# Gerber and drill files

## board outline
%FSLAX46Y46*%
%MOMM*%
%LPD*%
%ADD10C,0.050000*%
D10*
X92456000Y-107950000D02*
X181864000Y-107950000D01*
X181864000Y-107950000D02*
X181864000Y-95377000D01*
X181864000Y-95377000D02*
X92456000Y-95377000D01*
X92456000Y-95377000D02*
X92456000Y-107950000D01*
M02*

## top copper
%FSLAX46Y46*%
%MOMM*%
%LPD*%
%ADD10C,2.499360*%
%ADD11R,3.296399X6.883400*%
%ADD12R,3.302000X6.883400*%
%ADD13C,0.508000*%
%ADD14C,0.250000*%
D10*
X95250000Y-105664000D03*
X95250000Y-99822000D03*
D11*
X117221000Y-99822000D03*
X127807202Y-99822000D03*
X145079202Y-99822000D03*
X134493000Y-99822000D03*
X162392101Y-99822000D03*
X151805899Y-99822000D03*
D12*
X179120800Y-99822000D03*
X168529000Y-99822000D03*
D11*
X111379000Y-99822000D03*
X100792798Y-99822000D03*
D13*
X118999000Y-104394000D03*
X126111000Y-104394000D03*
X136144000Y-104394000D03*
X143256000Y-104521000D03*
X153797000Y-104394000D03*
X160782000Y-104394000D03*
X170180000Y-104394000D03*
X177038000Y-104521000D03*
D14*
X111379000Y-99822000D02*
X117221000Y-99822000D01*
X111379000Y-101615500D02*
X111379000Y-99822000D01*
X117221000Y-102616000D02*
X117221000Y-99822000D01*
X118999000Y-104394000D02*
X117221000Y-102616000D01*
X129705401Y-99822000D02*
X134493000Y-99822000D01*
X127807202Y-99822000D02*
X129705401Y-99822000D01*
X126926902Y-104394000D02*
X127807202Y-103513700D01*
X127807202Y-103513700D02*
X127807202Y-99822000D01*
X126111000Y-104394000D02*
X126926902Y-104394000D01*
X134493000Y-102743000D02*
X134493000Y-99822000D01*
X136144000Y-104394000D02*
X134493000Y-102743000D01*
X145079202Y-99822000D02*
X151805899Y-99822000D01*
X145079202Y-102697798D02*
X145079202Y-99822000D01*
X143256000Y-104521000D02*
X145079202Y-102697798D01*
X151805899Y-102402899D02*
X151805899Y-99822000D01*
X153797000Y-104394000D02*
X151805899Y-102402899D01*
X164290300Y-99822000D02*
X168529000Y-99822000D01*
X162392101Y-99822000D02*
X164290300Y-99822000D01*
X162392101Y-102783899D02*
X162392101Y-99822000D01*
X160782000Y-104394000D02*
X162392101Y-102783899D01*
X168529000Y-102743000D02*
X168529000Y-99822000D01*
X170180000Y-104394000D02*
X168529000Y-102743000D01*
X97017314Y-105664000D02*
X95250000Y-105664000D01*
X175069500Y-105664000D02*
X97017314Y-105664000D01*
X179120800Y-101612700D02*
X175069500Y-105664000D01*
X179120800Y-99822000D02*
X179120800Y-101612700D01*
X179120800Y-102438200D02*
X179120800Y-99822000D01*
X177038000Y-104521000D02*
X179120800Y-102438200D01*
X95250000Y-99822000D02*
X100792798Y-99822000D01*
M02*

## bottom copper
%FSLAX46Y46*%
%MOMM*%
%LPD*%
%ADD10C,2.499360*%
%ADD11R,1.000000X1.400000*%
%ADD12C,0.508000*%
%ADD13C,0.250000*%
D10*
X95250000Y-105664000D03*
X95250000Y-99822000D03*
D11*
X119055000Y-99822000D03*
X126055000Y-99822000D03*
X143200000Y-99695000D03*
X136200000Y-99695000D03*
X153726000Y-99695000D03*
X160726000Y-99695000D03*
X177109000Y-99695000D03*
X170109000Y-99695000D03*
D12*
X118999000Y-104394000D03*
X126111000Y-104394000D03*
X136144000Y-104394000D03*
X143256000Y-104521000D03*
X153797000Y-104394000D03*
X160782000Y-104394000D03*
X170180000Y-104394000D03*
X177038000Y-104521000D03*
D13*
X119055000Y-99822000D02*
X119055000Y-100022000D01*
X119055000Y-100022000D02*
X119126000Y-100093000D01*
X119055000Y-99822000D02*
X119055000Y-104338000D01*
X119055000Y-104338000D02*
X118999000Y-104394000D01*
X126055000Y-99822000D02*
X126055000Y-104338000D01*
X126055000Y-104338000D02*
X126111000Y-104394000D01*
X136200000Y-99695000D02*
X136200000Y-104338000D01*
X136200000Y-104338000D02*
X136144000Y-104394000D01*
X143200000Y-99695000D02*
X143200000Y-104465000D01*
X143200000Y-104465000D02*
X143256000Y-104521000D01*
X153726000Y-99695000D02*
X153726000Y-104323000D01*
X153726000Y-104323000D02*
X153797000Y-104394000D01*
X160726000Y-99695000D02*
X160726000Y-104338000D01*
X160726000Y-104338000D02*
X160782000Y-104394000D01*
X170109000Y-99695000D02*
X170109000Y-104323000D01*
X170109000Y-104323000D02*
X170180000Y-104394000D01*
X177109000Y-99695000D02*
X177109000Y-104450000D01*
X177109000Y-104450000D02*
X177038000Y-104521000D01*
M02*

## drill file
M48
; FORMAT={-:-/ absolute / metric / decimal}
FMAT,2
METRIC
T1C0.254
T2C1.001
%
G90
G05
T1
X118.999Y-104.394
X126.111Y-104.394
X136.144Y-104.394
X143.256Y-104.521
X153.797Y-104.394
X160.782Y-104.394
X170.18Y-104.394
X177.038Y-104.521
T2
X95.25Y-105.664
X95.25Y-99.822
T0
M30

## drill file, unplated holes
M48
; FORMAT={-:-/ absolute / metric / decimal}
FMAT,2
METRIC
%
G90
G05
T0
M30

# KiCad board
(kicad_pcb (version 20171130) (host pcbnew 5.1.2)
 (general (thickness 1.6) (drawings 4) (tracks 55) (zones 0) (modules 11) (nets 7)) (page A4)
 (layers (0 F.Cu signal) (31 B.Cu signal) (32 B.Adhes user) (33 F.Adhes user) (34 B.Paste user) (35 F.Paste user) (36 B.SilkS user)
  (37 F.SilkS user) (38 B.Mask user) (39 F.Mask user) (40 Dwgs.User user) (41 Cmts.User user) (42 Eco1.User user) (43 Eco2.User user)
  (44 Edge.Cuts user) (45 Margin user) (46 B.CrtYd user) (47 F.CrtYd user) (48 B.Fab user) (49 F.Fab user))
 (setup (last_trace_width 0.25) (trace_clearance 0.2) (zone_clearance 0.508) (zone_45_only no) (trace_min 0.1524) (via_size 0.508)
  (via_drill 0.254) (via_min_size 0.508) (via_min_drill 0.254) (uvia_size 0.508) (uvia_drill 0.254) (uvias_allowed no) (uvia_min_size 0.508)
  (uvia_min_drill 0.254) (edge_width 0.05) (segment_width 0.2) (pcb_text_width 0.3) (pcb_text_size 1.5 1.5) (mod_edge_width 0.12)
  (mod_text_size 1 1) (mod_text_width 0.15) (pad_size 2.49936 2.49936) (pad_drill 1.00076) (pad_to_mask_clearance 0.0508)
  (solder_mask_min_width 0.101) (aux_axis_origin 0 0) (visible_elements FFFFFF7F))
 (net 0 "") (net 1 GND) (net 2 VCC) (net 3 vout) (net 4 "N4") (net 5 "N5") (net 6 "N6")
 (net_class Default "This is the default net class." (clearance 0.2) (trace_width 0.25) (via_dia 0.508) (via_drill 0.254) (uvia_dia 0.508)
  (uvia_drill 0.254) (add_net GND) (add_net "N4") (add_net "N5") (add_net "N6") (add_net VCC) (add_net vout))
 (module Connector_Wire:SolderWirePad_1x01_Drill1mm (layer F.Cu) (at 95.25 105.664)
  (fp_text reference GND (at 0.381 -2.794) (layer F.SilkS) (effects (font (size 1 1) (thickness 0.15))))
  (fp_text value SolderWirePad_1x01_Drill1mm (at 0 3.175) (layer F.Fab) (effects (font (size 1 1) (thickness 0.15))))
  (pad 1 thru_hole circle (at 0 0) (size 2.49936 2.49936) (drill 1.00076) (layers *.Cu *.Mask) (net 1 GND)))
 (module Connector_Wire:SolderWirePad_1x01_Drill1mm (layer F.Cu) (at 95.25 99.822)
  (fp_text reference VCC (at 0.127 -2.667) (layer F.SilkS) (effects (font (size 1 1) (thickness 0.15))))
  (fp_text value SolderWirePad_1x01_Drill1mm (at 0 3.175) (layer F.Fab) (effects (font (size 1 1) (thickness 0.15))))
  (pad 1 thru_hole circle (at 0 0) (size 2.49936 2.49936) (drill 1.00076) (layers *.Cu *.Mask) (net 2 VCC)))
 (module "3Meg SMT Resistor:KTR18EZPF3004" (layer F.Cu) (at 122.514101 99.822 180)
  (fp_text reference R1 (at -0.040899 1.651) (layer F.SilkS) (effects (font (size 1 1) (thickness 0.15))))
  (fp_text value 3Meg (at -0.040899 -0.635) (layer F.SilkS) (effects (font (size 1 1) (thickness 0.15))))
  (pad 2 smd rect (at 5.293101 0 180) (size 3.296399 6.8834) (layers F.Cu F.Paste F.Mask) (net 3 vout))
  (pad 1 smd rect (at -5.293101 0 180) (size 3.296399 6.8834) (layers F.Cu F.Paste F.Mask) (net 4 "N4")))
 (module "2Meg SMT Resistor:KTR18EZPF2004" (layer F.Cu) (at 139.786101 99.822 180)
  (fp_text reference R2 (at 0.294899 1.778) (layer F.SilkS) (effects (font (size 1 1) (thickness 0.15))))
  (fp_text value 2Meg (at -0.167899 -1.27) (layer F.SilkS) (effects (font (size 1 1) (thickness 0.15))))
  (pad 1 smd rect (at -5.293101 0 180) (size 3.296399 6.8834) (layers F.Cu F.Paste F.Mask) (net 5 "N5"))
  (pad 2 smd rect (at 5.293101 0 180) (size 3.296399 6.8834) (layers F.Cu F.Paste F.Mask) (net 4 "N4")))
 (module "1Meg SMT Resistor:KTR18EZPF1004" (layer F.Cu) (at 157.099 99.822 180)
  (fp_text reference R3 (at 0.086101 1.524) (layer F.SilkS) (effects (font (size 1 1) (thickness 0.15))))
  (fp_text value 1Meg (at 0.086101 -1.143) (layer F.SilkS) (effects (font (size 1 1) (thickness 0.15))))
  (pad 1 smd rect (at -5.293101 0 180) (size 3.296399 6.8834) (layers F.Cu F.Paste F.Mask) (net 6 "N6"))
  (pad 2 smd rect (at 5.293101 0 180) (size 3.296399 6.8834) (layers F.Cu F.Paste F.Mask) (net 5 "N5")))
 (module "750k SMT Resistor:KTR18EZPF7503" (layer F.Cu) (at 173.8249 99.822 180)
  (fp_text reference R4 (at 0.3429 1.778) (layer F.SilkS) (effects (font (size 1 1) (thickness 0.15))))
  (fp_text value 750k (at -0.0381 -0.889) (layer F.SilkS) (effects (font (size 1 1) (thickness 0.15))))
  (pad 1 smd rect (at -5.2959 0 180) (size 3.302 6.8834) (layers F.Cu F.Paste F.Mask) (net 1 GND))
  (pad 2 smd rect (at 5.2959 0 180) (size 3.302 6.8834) (layers F.Cu F.Paste F.Mask) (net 6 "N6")))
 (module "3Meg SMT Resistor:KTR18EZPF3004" (layer F.Cu) (at 106.085899 99.822 180)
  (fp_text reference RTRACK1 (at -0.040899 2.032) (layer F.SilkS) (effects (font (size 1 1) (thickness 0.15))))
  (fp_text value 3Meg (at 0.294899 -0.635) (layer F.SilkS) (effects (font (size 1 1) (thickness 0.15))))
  (pad 1 smd rect (at -5.293101 0 180) (size 3.296399 6.8834) (layers F.Cu F.Paste F.Mask) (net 3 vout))
  (pad 2 smd rect (at 5.293101 0 180) (size 3.296399 6.8834) (layers F.Cu F.Paste F.Mask) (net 2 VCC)))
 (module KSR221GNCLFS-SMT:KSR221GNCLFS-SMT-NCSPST (layer B.Cu) (at 122.555 99.822)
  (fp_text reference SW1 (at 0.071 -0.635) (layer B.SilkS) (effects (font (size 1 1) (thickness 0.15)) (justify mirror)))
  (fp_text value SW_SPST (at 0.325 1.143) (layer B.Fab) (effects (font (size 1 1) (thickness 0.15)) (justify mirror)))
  (pad 1 smd rect (at -3.5 0) (size 1 1.4) (layers B.Cu B.Paste B.Mask) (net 3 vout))
  (pad 2 smd rect (at 3.5 0) (size 1 1.4) (layers B.Cu B.Paste B.Mask) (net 4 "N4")))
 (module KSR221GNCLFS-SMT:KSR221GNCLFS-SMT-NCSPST (layer B.Cu) (at 139.7 99.695)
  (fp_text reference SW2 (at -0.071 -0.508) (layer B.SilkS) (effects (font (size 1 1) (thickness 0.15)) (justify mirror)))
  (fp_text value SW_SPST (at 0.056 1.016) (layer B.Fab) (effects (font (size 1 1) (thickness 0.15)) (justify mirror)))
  (pad 2 smd rect (at 3.5 0) (size 1 1.4) (layers B.Cu B.Paste B.Mask) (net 5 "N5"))
  (pad 1 smd rect (at -3.5 0) (size 1 1.4) (layers B.Cu B.Paste B.Mask) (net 4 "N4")))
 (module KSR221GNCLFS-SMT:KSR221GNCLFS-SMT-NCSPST (layer B.Cu) (at 157.226 99.695)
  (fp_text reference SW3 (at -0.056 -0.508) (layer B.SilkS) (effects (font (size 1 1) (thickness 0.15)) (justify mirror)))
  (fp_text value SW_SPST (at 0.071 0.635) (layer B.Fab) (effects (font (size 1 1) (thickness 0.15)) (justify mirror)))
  (pad 1 smd rect (at -3.5 0) (size 1 1.4) (layers B.Cu B.Paste B.Mask) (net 5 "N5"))
  (pad 2 smd rect (at 3.5 0) (size 1 1.4) (layers B.Cu B.Paste B.Mask) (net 6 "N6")))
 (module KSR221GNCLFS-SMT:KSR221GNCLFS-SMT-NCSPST (layer B.Cu) (at 173.609 99.695)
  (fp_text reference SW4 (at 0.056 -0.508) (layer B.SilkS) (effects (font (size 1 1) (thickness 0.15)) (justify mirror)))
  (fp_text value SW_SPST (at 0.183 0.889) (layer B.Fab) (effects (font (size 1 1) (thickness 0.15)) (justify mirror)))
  (pad 2 smd rect (at 3.5 0) (size 1 1.4) (layers B.Cu B.Paste B.Mask) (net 1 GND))
  (pad 1 smd rect (at -3.5 0) (size 1 1.4) (layers B.Cu B.Paste B.Mask) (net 6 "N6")))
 (gr_line (start 92.456 107.95) (end 181.864 107.95) (layer Edge.Cuts) (width 0.05))
 (gr_line (start 181.864 107.95) (end 181.864 95.377) (layer Edge.Cuts) (width 0.05))
 (gr_line (start 181.864 95.377) (end 92.456 95.377) (layer Edge.Cuts) (width 0.05))
 (gr_line (start 92.456 95.377) (end 92.456 107.95) (layer Edge.Cuts) (width 0.05))
 (segment (start 111.379 99.822) (end 117.221 99.822) (width 0.25) (layer F.Cu) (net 3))
 (segment (start 119.055 99.822) (end 119.055 100.022) (width 0.25) (layer B.Cu) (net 3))
 (segment (start 119.055 100.022) (end 119.126 100.093) (width 0.25) (layer B.Cu) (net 3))
 (segment (start 111.379 101.6155) (end 111.379 99.822) (width 0.25) (layer F.Cu) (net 3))
 (via (at 118.999 104.394) (size 0.508) (drill 0.254) (layers F.Cu B.Cu) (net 3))
 (segment (start 119.055 99.822) (end 119.055 104.338) (width 0.25) (layer B.Cu) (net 3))
 (segment (start 119.055 104.338) (end 118.999 104.394) (width 0.25) (layer B.Cu) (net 3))
 (segment (start 117.221 102.616) (end 117.221 99.822) (width 0.25) (layer F.Cu) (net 3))
 (segment (start 118.999 104.394) (end 117.221 102.616) (width 0.25) (layer F.Cu) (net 3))
 (segment (start 129.705401 99.822) (end 134.493 99.822) (width 0.25) (layer F.Cu) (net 4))
 (segment (start 127.807202 99.822) (end 129.705401 99.822) (width 0.25) (layer F.Cu) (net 4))
 (via (at 126.111 104.394) (size 0.508) (drill 0.254) (layers F.Cu B.Cu) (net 4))
 (segment (start 126.055 99.822) (end 126.055 104.338) (width 0.25) (layer B.Cu) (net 4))
 (segment (start 126.055 104.338) (end 126.111 104.394) (width 0.25) (layer B.Cu) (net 4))
 (segment (start 126.926902 104.394) (end 127.807202 103.5137) (width 0.25) (layer F.Cu) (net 4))
 (segment (start 127.807202 103.5137) (end 127.807202 99.822) (width 0.25) (layer F.Cu) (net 4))
 (segment (start 126.111 104.394) (end 126.926902 104.394) (width 0.25) (layer F.Cu) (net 4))
 (via (at 136.144 104.394) (size 0.508) (drill 0.254) (layers F.Cu B.Cu) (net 4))
 (segment (start 136.2 99.695) (end 136.2 104.338) (width 0.25) (layer B.Cu) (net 4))
 (segment (start 136.2 104.338) (end 136.144 104.394) (width 0.25) (layer B.Cu) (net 4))
 (segment (start 134.493 102.743) (end 134.493 99.822) (width 0.25) (layer F.Cu) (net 4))
 (segment (start 136.144 104.394) (end 134.493 102.743) (width 0.25) (layer F.Cu) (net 4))
 (segment (start 145.079202 99.822) (end 151.805899 99.822) (width 0.25) (layer F.Cu) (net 5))
 (segment (start 143.2 99.695) (end 143.2 104.465) (width 0.25) (layer B.Cu) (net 5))
 (via (at 143.256 104.521) (size 0.508) (drill 0.254) (layers F.Cu B.Cu) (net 5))
 (segment (start 143.2 104.465) (end 143.256 104.521) (width 0.25) (layer B.Cu) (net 5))
 (segment (start 145.079202 102.697798) (end 145.079202 99.822) (width 0.25) (layer F.Cu) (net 5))
 (segment (start 143.256 104.521) (end 145.079202 102.697798) (width 0.25) (layer F.Cu) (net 5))
 (via (at 153.797 104.394) (size 0.508) (drill 0.254) (layers F.Cu B.Cu) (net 5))
 (segment (start 153.726 99.695) (end 153.726 104.323) (width 0.25) (layer B.Cu) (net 5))
 (segment (start 153.726 104.323) (end 153.797 104.394) (width 0.25) (layer B.Cu) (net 5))
 (segment (start 151.805899 102.402899) (end 151.805899 99.822) (width 0.25) (layer F.Cu) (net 5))
 (segment (start 153.797 104.394) (end 151.805899 102.402899) (width 0.25) (layer F.Cu) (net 5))
 (segment (start 164.2903 99.822) (end 168.529 99.822) (width 0.25) (layer F.Cu) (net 6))
 (segment (start 162.392101 99.822) (end 164.2903 99.822) (width 0.25) (layer F.Cu) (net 6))
 (via (at 160.782 104.394) (size 0.508) (drill 0.254) (layers F.Cu B.Cu) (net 6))
 (segment (start 160.726 99.695) (end 160.726 104.338) (width 0.25) (layer B.Cu) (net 6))
 (segment (start 160.726 104.338) (end 160.782 104.394) (width 0.25) (layer B.Cu) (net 6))
 (segment (start 162.392101 102.783899) (end 162.392101 99.822) (width 0.25) (layer F.Cu) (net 6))
 (segment (start 160.782 104.394) (end 162.392101 102.783899) (width 0.25) (layer F.Cu) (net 6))
 (via (at 170.18 104.394) (size 0.508) (drill 0.254) (layers F.Cu B.Cu) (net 6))
 (segment (start 170.109 99.695) (end 170.109 104.323) (width 0.25) (layer B.Cu) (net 6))
 (segment (start 170.109 104.323) (end 170.18 104.394) (width 0.25) (layer B.Cu) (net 6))
 (segment (start 168.529 102.743) (end 168.529 99.822) (width 0.25) (layer F.Cu) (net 6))
 (segment (start 170.18 104.394) (end 168.529 102.743) (width 0.25) (layer F.Cu) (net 6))
 (segment (start 97.017314 105.664) (end 95.25 105.664) (width 0.25) (layer F.Cu) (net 1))
 (segment (start 175.0695 105.664) (end 97.017314 105.664) (width 0.25) (layer F.Cu) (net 1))
 (segment (start 179.1208 101.6127) (end 175.0695 105.664) (width 0.25) (layer F.Cu) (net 1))
 (segment (start 179.1208 99.822) (end 179.1208 101.6127) (width 0.25) (layer F.Cu) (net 1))
 (via (at 177.038 104.521) (size 0.508) (drill 0.254) (layers F.Cu B.Cu) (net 1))
 (segment (start 177.109 99.695) (end 177.109 104.45) (width 0.25) (layer B.Cu) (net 1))
 (segment (start 177.109 104.45) (end 177.038 104.521) (width 0.25) (layer B.Cu) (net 1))
 (segment (start 179.1208 102.4382) (end 179.1208 99.822) (width 0.25) (layer F.Cu) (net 1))
 (segment (start 177.038 104.521) (end 179.1208 102.4382) (width 0.25) (layer F.Cu) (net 1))
 (segment (start 95.25 99.822) (end 100.792798 99.822) (width 0.25) (layer F.Cu) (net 2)))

